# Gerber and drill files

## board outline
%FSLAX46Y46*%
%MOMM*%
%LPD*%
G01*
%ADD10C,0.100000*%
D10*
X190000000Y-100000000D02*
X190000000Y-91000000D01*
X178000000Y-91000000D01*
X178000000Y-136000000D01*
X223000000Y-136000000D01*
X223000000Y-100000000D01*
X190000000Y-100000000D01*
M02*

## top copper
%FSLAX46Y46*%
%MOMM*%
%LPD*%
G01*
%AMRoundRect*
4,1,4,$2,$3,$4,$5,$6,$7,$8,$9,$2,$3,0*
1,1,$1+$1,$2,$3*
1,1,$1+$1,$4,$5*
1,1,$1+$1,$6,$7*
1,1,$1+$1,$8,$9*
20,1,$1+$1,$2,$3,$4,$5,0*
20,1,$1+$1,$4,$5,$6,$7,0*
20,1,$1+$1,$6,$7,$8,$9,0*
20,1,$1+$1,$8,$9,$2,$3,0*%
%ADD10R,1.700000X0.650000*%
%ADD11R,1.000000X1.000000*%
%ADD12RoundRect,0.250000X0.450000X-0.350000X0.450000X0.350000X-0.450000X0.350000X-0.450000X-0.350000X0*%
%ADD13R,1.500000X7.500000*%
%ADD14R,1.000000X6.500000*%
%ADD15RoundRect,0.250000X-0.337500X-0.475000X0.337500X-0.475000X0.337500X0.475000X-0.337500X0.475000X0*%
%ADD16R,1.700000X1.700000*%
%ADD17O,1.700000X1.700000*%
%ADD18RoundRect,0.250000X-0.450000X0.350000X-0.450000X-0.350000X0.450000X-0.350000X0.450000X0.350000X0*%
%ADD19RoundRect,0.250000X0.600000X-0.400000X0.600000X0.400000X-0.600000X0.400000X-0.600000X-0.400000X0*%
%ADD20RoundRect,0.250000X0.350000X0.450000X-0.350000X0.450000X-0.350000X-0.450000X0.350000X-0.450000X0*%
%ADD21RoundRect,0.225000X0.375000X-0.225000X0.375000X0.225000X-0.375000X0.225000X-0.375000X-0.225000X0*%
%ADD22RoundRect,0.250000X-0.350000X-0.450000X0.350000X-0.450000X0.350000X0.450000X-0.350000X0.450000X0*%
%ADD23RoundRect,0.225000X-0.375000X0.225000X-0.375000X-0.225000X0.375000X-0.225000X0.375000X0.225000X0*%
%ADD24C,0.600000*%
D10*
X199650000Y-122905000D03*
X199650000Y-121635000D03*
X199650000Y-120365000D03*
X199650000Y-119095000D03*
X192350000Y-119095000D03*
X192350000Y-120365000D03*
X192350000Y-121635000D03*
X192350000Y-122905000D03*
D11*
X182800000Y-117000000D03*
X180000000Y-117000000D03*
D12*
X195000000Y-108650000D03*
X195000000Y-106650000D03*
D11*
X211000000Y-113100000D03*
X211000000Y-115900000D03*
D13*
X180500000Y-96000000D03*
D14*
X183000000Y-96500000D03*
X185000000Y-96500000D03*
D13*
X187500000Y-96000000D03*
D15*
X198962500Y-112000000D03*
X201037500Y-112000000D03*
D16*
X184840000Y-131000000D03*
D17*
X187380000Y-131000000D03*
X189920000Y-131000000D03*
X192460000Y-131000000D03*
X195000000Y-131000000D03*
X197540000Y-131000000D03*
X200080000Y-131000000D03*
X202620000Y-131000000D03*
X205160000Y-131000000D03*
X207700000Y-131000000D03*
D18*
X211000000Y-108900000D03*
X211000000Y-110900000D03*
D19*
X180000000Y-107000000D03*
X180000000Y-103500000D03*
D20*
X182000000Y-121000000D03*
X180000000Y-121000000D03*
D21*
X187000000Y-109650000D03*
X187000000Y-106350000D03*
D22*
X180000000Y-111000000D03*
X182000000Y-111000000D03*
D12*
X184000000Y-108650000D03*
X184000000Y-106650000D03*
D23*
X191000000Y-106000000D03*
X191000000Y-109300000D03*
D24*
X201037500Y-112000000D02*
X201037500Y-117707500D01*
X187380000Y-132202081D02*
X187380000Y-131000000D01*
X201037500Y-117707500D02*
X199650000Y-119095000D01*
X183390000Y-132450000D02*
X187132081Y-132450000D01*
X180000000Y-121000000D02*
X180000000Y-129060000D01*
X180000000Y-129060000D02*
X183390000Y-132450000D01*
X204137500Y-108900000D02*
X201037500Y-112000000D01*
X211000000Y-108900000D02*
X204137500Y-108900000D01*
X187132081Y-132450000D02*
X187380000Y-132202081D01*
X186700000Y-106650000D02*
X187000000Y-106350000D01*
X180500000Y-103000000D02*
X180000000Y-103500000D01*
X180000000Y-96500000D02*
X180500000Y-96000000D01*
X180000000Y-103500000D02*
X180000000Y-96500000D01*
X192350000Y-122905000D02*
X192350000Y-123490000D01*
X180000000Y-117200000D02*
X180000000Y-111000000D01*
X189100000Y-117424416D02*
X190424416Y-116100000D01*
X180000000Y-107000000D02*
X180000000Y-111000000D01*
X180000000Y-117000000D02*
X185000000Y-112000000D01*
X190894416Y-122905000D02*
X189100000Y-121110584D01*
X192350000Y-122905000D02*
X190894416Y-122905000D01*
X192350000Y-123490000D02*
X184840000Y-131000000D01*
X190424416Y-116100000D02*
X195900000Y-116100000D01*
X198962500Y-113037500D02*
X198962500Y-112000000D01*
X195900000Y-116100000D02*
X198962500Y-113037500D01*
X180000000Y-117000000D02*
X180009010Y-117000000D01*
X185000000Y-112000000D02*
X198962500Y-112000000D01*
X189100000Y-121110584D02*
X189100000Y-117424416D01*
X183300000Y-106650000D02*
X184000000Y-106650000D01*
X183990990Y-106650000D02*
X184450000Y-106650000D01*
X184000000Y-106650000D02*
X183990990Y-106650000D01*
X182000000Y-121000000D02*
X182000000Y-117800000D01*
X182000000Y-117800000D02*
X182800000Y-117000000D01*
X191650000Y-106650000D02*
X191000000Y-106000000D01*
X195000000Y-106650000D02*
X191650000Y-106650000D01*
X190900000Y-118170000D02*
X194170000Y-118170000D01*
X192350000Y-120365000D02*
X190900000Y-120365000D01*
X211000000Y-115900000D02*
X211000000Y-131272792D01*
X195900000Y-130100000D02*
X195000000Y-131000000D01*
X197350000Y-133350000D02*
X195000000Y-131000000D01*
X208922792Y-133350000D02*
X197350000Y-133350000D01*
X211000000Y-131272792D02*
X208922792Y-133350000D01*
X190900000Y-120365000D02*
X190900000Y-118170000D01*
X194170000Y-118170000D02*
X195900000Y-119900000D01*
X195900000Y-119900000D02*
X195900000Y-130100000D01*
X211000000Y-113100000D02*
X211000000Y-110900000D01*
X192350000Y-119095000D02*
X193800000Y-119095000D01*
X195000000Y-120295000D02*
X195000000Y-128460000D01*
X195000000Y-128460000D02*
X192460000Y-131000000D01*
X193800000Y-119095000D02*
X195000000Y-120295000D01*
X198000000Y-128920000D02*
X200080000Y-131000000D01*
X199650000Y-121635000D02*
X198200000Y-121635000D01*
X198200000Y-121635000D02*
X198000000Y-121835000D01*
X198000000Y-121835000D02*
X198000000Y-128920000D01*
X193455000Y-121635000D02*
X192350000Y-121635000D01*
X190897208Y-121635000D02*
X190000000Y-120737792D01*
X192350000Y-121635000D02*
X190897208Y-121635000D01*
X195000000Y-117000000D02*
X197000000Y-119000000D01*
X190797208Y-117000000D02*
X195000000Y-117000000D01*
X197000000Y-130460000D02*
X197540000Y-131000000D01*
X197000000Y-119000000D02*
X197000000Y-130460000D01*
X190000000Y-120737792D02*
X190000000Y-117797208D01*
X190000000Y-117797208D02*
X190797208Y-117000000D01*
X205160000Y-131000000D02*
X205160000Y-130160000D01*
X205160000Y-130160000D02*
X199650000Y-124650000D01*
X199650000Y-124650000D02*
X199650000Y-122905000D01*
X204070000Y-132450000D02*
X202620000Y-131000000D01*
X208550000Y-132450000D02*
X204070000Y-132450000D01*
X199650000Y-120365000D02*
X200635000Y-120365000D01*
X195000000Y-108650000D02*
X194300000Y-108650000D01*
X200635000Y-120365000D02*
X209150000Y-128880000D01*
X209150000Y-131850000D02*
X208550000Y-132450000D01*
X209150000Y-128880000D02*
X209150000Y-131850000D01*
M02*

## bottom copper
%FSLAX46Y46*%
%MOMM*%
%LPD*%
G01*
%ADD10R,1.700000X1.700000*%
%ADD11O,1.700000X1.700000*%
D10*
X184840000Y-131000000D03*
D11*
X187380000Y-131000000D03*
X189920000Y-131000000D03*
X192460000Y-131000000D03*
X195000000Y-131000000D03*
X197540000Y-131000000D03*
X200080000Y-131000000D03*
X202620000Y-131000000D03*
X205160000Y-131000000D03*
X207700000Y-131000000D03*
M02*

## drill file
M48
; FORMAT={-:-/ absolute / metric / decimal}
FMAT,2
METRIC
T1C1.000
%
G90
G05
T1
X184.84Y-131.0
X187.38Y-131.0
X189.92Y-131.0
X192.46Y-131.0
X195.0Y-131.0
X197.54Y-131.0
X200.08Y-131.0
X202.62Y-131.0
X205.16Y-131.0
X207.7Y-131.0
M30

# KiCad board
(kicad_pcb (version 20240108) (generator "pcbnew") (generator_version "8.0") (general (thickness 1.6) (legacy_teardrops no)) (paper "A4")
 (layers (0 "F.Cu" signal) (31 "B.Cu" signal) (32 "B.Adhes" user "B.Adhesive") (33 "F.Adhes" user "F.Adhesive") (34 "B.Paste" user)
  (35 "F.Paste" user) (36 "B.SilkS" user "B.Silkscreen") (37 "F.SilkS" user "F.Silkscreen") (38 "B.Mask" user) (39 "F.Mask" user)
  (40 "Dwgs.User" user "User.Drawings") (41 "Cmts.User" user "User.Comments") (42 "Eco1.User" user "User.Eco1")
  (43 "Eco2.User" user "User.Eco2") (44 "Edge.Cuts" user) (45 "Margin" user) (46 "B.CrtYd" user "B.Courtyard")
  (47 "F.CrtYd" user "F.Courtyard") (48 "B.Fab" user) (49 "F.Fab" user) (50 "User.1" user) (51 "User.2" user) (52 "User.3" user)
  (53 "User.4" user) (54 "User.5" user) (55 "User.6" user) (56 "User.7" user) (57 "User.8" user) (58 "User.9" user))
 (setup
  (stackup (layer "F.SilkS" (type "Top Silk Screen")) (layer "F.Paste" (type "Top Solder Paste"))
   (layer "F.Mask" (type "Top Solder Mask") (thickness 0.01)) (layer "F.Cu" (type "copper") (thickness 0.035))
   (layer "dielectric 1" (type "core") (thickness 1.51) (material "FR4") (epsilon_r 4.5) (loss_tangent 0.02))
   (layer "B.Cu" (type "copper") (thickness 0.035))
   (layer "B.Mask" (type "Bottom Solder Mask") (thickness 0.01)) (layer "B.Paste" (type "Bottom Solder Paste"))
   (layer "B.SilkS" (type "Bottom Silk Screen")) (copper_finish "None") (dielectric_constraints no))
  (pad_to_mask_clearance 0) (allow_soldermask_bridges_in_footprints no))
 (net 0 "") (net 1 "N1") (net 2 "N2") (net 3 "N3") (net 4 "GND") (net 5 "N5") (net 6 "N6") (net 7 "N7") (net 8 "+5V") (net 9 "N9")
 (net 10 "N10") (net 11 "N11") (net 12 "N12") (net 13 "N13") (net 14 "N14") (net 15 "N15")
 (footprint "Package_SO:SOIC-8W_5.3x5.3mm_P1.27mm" (layer "F.Cu") (at 196 121 180)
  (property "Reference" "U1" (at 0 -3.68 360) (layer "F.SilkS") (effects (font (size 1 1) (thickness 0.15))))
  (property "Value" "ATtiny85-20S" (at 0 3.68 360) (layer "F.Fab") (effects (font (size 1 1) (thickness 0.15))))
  (pad "1" smd rect (at -3.65 -1.905 180) (size 1.7 0.65) (layers "F.Cu" "F.Paste" "F.Mask") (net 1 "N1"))
  (pad "2" smd rect (at -3.65 -0.635 180) (size 1.7 0.65) (layers "F.Cu" "F.Paste" "F.Mask") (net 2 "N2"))
  (pad "3" smd rect (at -3.65 0.635 180) (size 1.7 0.65) (layers "F.Cu" "F.Paste" "F.Mask") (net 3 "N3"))
  (pad "4" smd rect (at -3.65 1.905 180) (size 1.7 0.65) (layers "F.Cu" "F.Paste" "F.Mask") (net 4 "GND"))
  (pad "5" smd rect (at 3.65 1.905 180) (size 1.7 0.65) (layers "F.Cu" "F.Paste" "F.Mask") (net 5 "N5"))
  (pad "6" smd rect (at 3.65 0.635 180) (size 1.7 0.65) (layers "F.Cu" "F.Paste" "F.Mask") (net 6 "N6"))
  (pad "7" smd rect (at 3.65 -0.635 180) (size 1.7 0.65) (layers "F.Cu" "F.Paste" "F.Mask") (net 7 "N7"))
  (pad "8" smd rect (at 3.65 -1.905 180) (size 1.7 0.65) (layers "F.Cu" "F.Paste" "F.Mask") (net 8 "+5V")))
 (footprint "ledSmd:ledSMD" (layer "F.Cu") (at 181 117 180)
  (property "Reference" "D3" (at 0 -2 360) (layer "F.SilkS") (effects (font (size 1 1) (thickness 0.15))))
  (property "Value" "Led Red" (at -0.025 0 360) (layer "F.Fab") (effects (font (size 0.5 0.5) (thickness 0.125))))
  (pad "1" smd rect (at -1.8 0 180) (size 1 1) (layers "F.Cu" "F.Paste" "F.Mask") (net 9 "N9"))
  (pad "2" smd rect (at 1 0 180) (size 1 1) (layers "F.Cu" "F.Paste" "F.Mask") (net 8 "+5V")))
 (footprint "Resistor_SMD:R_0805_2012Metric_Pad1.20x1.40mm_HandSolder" (layer "F.Cu") (at 195 107.65 90)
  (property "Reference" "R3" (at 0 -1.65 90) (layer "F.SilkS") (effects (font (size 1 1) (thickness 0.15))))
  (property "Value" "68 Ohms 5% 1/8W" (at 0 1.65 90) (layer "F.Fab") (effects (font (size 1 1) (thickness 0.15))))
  (pad "1" smd roundrect (at -1 0 90) (size 1.2 1.4) (layers "F.Cu" "F.Paste" "F.Mask") (roundrect_rratio 0.208333) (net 3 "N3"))
  (pad "2" smd roundrect (at 1 0 90) (size 1.2 1.4) (layers "F.Cu" "F.Paste" "F.Mask") (roundrect_rratio 0.208333) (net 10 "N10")))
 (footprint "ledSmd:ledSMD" (layer "F.Cu") (at 211 114.9 -90)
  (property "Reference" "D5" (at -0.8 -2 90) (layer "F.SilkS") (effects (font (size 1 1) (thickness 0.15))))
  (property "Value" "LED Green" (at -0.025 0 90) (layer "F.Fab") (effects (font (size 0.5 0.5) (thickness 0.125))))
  (pad "1" smd rect (at -1.8 0 270) (size 1 1) (layers "F.Cu" "F.Paste" "F.Mask") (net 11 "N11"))
  (pad "2" smd rect (at 1 0 270) (size 1 1) (layers "F.Cu" "F.Paste" "F.Mask") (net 6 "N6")))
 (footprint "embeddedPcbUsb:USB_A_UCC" (layer "F.Cu") (at 184 96.2 -90)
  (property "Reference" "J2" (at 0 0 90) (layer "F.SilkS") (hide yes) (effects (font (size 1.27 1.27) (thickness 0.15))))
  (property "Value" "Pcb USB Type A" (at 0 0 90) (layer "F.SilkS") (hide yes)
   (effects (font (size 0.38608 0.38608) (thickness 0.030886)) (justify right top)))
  (pad "1" smd rect (at -0.2 3.5 270) (size 7.5 1.5) (layers "F.Cu" "F.Paste" "F.Mask") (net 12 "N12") (solder_mask_margin 0.1016))
  (pad "2" smd rect (at 0.3 1 270) (size 6.5 1) (layers "F.Cu" "F.Paste" "F.Mask") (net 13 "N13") (solder_mask_margin 0.1016))
  (pad "3" smd rect (at 0.3 -1 270) (size 6.5 1) (layers "F.Cu" "F.Paste" "F.Mask") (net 10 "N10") (solder_mask_margin 0.1016))
  (pad "4" smd rect (at -0.2 -3.5 270) (size 7.5 1.5) (layers "F.Cu" "F.Paste" "F.Mask") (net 4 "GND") (solder_mask_margin 0.1016)))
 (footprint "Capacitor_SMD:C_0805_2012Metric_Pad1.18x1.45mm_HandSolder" (layer "F.Cu") (at 200 112)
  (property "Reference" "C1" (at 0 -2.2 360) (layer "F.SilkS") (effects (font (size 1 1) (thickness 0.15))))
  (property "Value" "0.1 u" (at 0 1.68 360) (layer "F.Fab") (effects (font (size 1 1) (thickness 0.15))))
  (pad "1" smd roundrect (at -1.0375 0) (size 1.175 1.45) (layers "F.Cu" "F.Paste" "F.Mask") (roundrect_rratio 0.212766) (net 8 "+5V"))
  (pad "2" smd roundrect (at 1.0375 0) (size 1.175 1.45) (layers "F.Cu" "F.Paste" "F.Mask") (roundrect_rratio 0.212766) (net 4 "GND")))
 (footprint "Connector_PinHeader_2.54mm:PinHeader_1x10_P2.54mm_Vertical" (layer "F.Cu") (at 184.84 131 90)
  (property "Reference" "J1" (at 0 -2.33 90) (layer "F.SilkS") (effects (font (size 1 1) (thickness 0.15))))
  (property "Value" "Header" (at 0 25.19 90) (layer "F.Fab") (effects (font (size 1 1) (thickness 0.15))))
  (pad "1" thru_hole rect (at 0 0 90) (size 1.7 1.7) (drill 1) (layers "*.Cu" "*.Mask") (remove_unused_layers no) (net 8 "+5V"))
  (pad "2" thru_hole oval (at 0 2.54 90) (size 1.7 1.7) (drill 1) (layers "*.Cu" "*.Mask") (remove_unused_layers no) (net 4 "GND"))
  (pad "3" thru_hole oval (at 0 5.08 90) (size 1.7 1.7) (drill 1) (layers "*.Cu" "*.Mask") (remove_unused_layers no) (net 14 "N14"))
  (pad "4" thru_hole oval (at 0 7.62 90) (size 1.7 1.7) (drill 1) (layers "*.Cu" "*.Mask") (remove_unused_layers no) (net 5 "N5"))
  (pad "5" thru_hole oval (at 0 10.16 90) (size 1.7 1.7) (drill 1) (layers "*.Cu" "*.Mask") (remove_unused_layers no) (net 6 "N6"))
  (pad "6" thru_hole oval (at 0 12.7 90) (size 1.7 1.7) (drill 1) (layers "*.Cu" "*.Mask") (remove_unused_layers no) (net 7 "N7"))
  (pad "7" thru_hole oval (at 0 15.24 90) (size 1.7 1.7) (drill 1) (layers "*.Cu" "*.Mask") (remove_unused_layers no) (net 2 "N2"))
  (pad "8" thru_hole oval (at 0 17.78 90) (size 1.7 1.7) (drill 1) (layers "*.Cu" "*.Mask") (remove_unused_layers no) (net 3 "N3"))
  (pad "9" thru_hole oval (at 0 20.32 90) (size 1.7 1.7) (drill 1) (layers "*.Cu" "*.Mask") (remove_unused_layers no) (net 1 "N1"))
  (pad "10" thru_hole oval (at 0 22.86 90) (size 1.7 1.7) (drill 1) (layers "*.Cu" "*.Mask") (remove_unused_layers no) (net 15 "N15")))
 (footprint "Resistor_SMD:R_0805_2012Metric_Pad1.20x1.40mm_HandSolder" (layer "F.Cu") (at 211 109.9 -90)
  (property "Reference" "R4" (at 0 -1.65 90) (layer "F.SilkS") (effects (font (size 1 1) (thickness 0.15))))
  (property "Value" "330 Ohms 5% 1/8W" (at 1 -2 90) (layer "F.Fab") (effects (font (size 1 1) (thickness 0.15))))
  (pad "1" smd roundrect (at -1 0 270) (size 1.2 1.4) (layers "F.Cu" "F.Paste" "F.Mask") (roundrect_rratio 0.208333) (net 4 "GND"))
  (pad "2" smd roundrect (at 1 0 270) (size 1.2 1.4) (layers "F.Cu" "F.Paste" "F.Mask") (roundrect_rratio 0.208333) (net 11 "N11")))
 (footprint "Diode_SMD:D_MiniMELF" (layer "F.Cu") (at 180 105.25 90)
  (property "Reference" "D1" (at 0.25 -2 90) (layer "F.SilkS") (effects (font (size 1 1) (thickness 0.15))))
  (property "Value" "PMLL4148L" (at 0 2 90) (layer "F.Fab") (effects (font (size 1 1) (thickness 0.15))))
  (pad "1" smd roundrect (at -1.75 0 90) (size 1.3 1.7) (layers "F.Cu" "F.Paste" "F.Mask") (roundrect_rratio 0.1923076923) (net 8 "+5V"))
  (pad "2" smd roundrect (at 1.75 0 90) (size 1.3 1.7) (layers "F.Cu" "F.Paste" "F.Mask") (roundrect_rratio 0.1923076923) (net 12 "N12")))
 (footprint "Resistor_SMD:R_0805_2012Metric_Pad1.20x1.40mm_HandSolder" (layer "F.Cu") (at 181 121 180)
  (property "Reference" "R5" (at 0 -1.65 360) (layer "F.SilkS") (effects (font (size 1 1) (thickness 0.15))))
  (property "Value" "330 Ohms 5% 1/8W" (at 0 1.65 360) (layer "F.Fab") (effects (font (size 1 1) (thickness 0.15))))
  (pad "1" smd roundrect (at -1 0 180) (size 1.2 1.4) (layers "F.Cu" "F.Paste" "F.Mask") (roundrect_rratio 0.208333) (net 9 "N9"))
  (pad "2" smd roundrect (at 1 0 180) (size 1.2 1.4) (layers "F.Cu" "F.Paste" "F.Mask") (roundrect_rratio 0.208333) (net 4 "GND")))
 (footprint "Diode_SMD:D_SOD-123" (layer "F.Cu") (at 187 108 90)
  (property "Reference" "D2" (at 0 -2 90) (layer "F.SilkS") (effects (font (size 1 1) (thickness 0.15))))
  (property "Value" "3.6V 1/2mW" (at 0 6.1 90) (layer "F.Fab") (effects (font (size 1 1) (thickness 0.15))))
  (pad "1" smd roundrect (at -1.65 0 90) (size 0.9 1.2) (layers "F.Cu" "F.Paste" "F.Mask") (roundrect_rratio 0.25) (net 13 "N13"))
  (pad "2" smd roundrect (at 1.65 0 90) (size 0.9 1.2) (layers "F.Cu" "F.Paste" "F.Mask") (roundrect_rratio 0.25) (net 4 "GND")))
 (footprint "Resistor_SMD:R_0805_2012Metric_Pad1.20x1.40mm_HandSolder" (layer "F.Cu") (at 181 111)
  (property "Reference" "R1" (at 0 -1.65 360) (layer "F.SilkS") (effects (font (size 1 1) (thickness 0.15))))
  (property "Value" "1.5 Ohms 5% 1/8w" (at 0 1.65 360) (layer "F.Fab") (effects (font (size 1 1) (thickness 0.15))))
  (pad "1" smd roundrect (at -1 0) (size 1.2 1.4) (layers "F.Cu" "F.Paste" "F.Mask") (roundrect_rratio 0.208333) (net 8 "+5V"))
  (pad "2" smd roundrect (at 1 0) (size 1.2 1.4) (layers "F.Cu" "F.Paste" "F.Mask") (roundrect_rratio 0.208333) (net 13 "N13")))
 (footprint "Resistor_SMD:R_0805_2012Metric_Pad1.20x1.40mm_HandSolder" (layer "F.Cu") (at 184 107.65 90)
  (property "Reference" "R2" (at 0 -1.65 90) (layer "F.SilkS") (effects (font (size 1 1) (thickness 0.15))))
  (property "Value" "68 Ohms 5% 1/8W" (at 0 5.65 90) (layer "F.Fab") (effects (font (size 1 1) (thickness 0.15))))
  (pad "1" smd roundrect (at -1 0 90) (size 1.2 1.4) (layers "F.Cu" "F.Paste" "F.Mask") (roundrect_rratio 0.208333) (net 2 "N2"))
  (pad "2" smd roundrect (at 1 0 90) (size 1.2 1.4) (layers "F.Cu" "F.Paste" "F.Mask") (roundrect_rratio 0.208333) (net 13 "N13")))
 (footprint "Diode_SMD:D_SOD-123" (layer "F.Cu") (at 191 107.65 -90)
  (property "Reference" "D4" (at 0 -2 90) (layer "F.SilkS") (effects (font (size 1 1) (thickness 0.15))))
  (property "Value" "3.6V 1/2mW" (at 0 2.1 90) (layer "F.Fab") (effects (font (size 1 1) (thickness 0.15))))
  (pad "1" smd roundrect (at -1.65 0 270) (size 0.9 1.2) (layers "F.Cu" "F.Paste" "F.Mask") (roundrect_rratio 0.25) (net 10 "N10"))
  (pad "2" smd roundrect (at 1.65 0 270) (size 0.9 1.2) (layers "F.Cu" "F.Paste" "F.Mask") (roundrect_rratio 0.25) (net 4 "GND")))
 (gr_poly
  (pts (xy 190 100) (xy 190 91) (xy 178 91) (xy 178 136) (xy 223 136) (xy 223 100)) (stroke (width 0.1) (type solid)) (fill none)
  (layer "Edge.Cuts"))
 (segment (start 201.0375 112) (end 201.0375 117.7075) (width 0.6) (layer "F.Cu") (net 4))
 (segment (start 187.38 132.202081) (end 187.38 131) (width 0.6) (layer "F.Cu") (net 4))
 (segment (start 201.0375 117.7075) (end 199.65 119.095) (width 0.6) (layer "F.Cu") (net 4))
 (segment (start 183.39 132.45) (end 187.132081 132.45) (width 0.6) (layer "F.Cu") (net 4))
 (segment (start 180 121) (end 180 129.06) (width 0.6) (layer "F.Cu") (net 4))
 (segment (start 180 129.06) (end 183.39 132.45) (width 0.6) (layer "F.Cu") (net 4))
 (segment (start 204.1375 108.9) (end 201.0375 112) (width 0.6) (layer "F.Cu") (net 4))
 (segment (start 211 108.9) (end 204.1375 108.9) (width 0.6) (layer "F.Cu") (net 4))
 (segment (start 187.132081 132.45) (end 187.38 132.202081) (width 0.6) (layer "F.Cu") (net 4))
 (segment (start 186.7 106.65) (end 187 106.35) (width 0.6) (layer "F.Cu") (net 4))
 (segment (start 180.5 103) (end 180 103.5) (width 0.6) (layer "F.Cu") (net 12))
 (segment (start 180 96.5) (end 180.5 96) (width 0.6) (layer "F.Cu") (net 12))
 (segment (start 180 103.5) (end 180 96.5) (width 0.6) (layer "F.Cu") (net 12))
 (segment (start 192.35 122.905) (end 192.35 123.49) (width 0.6) (layer "F.Cu") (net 8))
 (segment (start 180 117.2) (end 180 111) (width 0.6) (layer "F.Cu") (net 8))
 (segment (start 189.1 117.424416) (end 190.424416 116.1) (width 0.6) (layer "F.Cu") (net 8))
 (segment (start 180 107) (end 180 111) (width 0.6) (layer "F.Cu") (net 8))
 (segment (start 180 117) (end 185 112) (width 0.6) (layer "F.Cu") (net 8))
 (segment (start 190.894416 122.905) (end 189.1 121.110584) (width 0.6) (layer "F.Cu") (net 8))
 (segment (start 192.35 122.905) (end 190.894416 122.905) (width 0.6) (layer "F.Cu") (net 8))
 (segment (start 192.35 123.49) (end 184.84 131) (width 0.6) (layer "F.Cu") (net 8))
 (segment (start 190.424416 116.1) (end 195.9 116.1) (width 0.6) (layer "F.Cu") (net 8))
 (segment (start 198.9625 113.0375) (end 198.9625 112) (width 0.6) (layer "F.Cu") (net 8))
 (segment (start 195.9 116.1) (end 198.9625 113.0375) (width 0.6) (layer "F.Cu") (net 8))
 (segment (start 180 117) (end 180.00901 117) (width 0.6) (layer "F.Cu") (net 8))
 (segment (start 185 112) (end 198.9625 112) (width 0.6) (layer "F.Cu") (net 8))
 (segment (start 189.1 121.110584) (end 189.1 117.424416) (width 0.6) (layer "F.Cu") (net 8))
 (segment (start 183.3 106.65) (end 184 106.65) (width 0.6) (layer "F.Cu") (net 13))
 (segment (start 183.99099 106.65) (end 184.45 106.65) (width 0.6) (layer "F.Cu") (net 13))
 (segment (start 184 106.65) (end 183.99099 106.65) (width 0.6) (layer "F.Cu") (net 13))
 (segment (start 182 121) (end 182 117.8) (width 0.6) (layer "F.Cu") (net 9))
 (segment (start 182 117.8) (end 182.8 117) (width 0.6) (layer "F.Cu") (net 9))
 (segment (start 191.65 106.65) (end 191 106) (width 0.6) (layer "F.Cu") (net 10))
 (segment (start 195 106.65) (end 191.65 106.65) (width 0.6) (layer "F.Cu") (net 10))
 (segment (start 190.9 118.17) (end 194.17 118.17) (width 0.6) (layer "F.Cu") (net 6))
 (segment (start 192.35 120.365) (end 190.9 120.365) (width 0.6) (layer "F.Cu") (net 6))
 (segment (start 211 115.9) (end 211 131.272792) (width 0.6) (layer "F.Cu") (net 6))
 (segment (start 195.9 130.1) (end 195 131) (width 0.6) (layer "F.Cu") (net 6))
 (segment (start 197.35 133.35) (end 195 131) (width 0.6) (layer "F.Cu") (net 6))
 (segment (start 208.922792 133.35) (end 197.35 133.35) (width 0.6) (layer "F.Cu") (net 6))
 (segment (start 211 131.272792) (end 208.922792 133.35) (width 0.6) (layer "F.Cu") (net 6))
 (segment (start 190.9 120.365) (end 190.9 118.17) (width 0.6) (layer "F.Cu") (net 6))
 (segment (start 194.17 118.17) (end 195.9 119.9) (width 0.6) (layer "F.Cu") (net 6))
 (segment (start 195.9 119.9) (end 195.9 130.1) (width 0.6) (layer "F.Cu") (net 6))
 (segment (start 211 113.1) (end 211 110.9) (width 0.6) (layer "F.Cu") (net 11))
 (segment (start 192.35 119.095) (end 193.8 119.095) (width 0.6) (layer "F.Cu") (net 5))
 (segment (start 195 120.295) (end 195 128.46) (width 0.6) (layer "F.Cu") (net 5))
 (segment (start 195 128.46) (end 192.46 131) (width 0.6) (layer "F.Cu") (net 5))
 (segment (start 193.8 119.095) (end 195 120.295) (width 0.6) (layer "F.Cu") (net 5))
 (segment (start 198 128.92) (end 200.08 131) (width 0.6) (layer "F.Cu") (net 2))
 (segment (start 199.65 121.635) (end 198.2 121.635) (width 0.6) (layer "F.Cu") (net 2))
 (segment (start 198.2 121.635) (end 198 121.835) (width 0.6) (layer "F.Cu") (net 2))
 (segment (start 198 121.835) (end 198 128.92) (width 0.6) (layer "F.Cu") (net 2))
 (segment (start 193.455 121.635) (end 192.35 121.635) (width 0.6) (layer "F.Cu") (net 7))
 (segment (start 190.897208 121.635) (end 190 120.737792) (width 0.6) (layer "F.Cu") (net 7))
 (segment (start 192.35 121.635) (end 190.897208 121.635) (width 0.6) (layer "F.Cu") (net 7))
 (segment (start 195 117) (end 197 119) (width 0.6) (layer "F.Cu") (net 7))
 (segment (start 190.797208 117) (end 195 117) (width 0.6) (layer "F.Cu") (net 7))
 (segment (start 197 130.46) (end 197.54 131) (width 0.6) (layer "F.Cu") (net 7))
 (segment (start 197 119) (end 197 130.46) (width 0.6) (layer "F.Cu") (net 7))
 (segment (start 190 120.737792) (end 190 117.797208) (width 0.6) (layer "F.Cu") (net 7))
 (segment (start 190 117.797208) (end 190.797208 117) (width 0.6) (layer "F.Cu") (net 7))
 (segment (start 205.16 131) (end 205.16 130.16) (width 0.6) (layer "F.Cu") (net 1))
 (segment (start 205.16 130.16) (end 199.65 124.65) (width 0.6) (layer "F.Cu") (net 1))
 (segment (start 199.65 124.65) (end 199.65 122.905) (width 0.6) (layer "F.Cu") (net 1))
 (segment (start 204.07 132.45) (end 202.62 131) (width 0.6) (layer "F.Cu") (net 3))
 (segment (start 208.55 132.45) (end 204.07 132.45) (width 0.6) (layer "F.Cu") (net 3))
 (segment (start 199.65 120.365) (end 200.635 120.365) (width 0.6) (layer "F.Cu") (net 3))
 (segment (start 195 108.65) (end 194.3 108.65) (width 0.6) (layer "F.Cu") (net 3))
 (segment (start 200.635 120.365) (end 209.15 128.88) (width 0.6) (layer "F.Cu") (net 3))
 (segment (start 209.15 131.85) (end 208.55 132.45) (width 0.6) (layer "F.Cu") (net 3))
 (segment (start 209.15 128.88) (end 209.15 131.85) (width 0.6) (layer "F.Cu") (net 3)))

